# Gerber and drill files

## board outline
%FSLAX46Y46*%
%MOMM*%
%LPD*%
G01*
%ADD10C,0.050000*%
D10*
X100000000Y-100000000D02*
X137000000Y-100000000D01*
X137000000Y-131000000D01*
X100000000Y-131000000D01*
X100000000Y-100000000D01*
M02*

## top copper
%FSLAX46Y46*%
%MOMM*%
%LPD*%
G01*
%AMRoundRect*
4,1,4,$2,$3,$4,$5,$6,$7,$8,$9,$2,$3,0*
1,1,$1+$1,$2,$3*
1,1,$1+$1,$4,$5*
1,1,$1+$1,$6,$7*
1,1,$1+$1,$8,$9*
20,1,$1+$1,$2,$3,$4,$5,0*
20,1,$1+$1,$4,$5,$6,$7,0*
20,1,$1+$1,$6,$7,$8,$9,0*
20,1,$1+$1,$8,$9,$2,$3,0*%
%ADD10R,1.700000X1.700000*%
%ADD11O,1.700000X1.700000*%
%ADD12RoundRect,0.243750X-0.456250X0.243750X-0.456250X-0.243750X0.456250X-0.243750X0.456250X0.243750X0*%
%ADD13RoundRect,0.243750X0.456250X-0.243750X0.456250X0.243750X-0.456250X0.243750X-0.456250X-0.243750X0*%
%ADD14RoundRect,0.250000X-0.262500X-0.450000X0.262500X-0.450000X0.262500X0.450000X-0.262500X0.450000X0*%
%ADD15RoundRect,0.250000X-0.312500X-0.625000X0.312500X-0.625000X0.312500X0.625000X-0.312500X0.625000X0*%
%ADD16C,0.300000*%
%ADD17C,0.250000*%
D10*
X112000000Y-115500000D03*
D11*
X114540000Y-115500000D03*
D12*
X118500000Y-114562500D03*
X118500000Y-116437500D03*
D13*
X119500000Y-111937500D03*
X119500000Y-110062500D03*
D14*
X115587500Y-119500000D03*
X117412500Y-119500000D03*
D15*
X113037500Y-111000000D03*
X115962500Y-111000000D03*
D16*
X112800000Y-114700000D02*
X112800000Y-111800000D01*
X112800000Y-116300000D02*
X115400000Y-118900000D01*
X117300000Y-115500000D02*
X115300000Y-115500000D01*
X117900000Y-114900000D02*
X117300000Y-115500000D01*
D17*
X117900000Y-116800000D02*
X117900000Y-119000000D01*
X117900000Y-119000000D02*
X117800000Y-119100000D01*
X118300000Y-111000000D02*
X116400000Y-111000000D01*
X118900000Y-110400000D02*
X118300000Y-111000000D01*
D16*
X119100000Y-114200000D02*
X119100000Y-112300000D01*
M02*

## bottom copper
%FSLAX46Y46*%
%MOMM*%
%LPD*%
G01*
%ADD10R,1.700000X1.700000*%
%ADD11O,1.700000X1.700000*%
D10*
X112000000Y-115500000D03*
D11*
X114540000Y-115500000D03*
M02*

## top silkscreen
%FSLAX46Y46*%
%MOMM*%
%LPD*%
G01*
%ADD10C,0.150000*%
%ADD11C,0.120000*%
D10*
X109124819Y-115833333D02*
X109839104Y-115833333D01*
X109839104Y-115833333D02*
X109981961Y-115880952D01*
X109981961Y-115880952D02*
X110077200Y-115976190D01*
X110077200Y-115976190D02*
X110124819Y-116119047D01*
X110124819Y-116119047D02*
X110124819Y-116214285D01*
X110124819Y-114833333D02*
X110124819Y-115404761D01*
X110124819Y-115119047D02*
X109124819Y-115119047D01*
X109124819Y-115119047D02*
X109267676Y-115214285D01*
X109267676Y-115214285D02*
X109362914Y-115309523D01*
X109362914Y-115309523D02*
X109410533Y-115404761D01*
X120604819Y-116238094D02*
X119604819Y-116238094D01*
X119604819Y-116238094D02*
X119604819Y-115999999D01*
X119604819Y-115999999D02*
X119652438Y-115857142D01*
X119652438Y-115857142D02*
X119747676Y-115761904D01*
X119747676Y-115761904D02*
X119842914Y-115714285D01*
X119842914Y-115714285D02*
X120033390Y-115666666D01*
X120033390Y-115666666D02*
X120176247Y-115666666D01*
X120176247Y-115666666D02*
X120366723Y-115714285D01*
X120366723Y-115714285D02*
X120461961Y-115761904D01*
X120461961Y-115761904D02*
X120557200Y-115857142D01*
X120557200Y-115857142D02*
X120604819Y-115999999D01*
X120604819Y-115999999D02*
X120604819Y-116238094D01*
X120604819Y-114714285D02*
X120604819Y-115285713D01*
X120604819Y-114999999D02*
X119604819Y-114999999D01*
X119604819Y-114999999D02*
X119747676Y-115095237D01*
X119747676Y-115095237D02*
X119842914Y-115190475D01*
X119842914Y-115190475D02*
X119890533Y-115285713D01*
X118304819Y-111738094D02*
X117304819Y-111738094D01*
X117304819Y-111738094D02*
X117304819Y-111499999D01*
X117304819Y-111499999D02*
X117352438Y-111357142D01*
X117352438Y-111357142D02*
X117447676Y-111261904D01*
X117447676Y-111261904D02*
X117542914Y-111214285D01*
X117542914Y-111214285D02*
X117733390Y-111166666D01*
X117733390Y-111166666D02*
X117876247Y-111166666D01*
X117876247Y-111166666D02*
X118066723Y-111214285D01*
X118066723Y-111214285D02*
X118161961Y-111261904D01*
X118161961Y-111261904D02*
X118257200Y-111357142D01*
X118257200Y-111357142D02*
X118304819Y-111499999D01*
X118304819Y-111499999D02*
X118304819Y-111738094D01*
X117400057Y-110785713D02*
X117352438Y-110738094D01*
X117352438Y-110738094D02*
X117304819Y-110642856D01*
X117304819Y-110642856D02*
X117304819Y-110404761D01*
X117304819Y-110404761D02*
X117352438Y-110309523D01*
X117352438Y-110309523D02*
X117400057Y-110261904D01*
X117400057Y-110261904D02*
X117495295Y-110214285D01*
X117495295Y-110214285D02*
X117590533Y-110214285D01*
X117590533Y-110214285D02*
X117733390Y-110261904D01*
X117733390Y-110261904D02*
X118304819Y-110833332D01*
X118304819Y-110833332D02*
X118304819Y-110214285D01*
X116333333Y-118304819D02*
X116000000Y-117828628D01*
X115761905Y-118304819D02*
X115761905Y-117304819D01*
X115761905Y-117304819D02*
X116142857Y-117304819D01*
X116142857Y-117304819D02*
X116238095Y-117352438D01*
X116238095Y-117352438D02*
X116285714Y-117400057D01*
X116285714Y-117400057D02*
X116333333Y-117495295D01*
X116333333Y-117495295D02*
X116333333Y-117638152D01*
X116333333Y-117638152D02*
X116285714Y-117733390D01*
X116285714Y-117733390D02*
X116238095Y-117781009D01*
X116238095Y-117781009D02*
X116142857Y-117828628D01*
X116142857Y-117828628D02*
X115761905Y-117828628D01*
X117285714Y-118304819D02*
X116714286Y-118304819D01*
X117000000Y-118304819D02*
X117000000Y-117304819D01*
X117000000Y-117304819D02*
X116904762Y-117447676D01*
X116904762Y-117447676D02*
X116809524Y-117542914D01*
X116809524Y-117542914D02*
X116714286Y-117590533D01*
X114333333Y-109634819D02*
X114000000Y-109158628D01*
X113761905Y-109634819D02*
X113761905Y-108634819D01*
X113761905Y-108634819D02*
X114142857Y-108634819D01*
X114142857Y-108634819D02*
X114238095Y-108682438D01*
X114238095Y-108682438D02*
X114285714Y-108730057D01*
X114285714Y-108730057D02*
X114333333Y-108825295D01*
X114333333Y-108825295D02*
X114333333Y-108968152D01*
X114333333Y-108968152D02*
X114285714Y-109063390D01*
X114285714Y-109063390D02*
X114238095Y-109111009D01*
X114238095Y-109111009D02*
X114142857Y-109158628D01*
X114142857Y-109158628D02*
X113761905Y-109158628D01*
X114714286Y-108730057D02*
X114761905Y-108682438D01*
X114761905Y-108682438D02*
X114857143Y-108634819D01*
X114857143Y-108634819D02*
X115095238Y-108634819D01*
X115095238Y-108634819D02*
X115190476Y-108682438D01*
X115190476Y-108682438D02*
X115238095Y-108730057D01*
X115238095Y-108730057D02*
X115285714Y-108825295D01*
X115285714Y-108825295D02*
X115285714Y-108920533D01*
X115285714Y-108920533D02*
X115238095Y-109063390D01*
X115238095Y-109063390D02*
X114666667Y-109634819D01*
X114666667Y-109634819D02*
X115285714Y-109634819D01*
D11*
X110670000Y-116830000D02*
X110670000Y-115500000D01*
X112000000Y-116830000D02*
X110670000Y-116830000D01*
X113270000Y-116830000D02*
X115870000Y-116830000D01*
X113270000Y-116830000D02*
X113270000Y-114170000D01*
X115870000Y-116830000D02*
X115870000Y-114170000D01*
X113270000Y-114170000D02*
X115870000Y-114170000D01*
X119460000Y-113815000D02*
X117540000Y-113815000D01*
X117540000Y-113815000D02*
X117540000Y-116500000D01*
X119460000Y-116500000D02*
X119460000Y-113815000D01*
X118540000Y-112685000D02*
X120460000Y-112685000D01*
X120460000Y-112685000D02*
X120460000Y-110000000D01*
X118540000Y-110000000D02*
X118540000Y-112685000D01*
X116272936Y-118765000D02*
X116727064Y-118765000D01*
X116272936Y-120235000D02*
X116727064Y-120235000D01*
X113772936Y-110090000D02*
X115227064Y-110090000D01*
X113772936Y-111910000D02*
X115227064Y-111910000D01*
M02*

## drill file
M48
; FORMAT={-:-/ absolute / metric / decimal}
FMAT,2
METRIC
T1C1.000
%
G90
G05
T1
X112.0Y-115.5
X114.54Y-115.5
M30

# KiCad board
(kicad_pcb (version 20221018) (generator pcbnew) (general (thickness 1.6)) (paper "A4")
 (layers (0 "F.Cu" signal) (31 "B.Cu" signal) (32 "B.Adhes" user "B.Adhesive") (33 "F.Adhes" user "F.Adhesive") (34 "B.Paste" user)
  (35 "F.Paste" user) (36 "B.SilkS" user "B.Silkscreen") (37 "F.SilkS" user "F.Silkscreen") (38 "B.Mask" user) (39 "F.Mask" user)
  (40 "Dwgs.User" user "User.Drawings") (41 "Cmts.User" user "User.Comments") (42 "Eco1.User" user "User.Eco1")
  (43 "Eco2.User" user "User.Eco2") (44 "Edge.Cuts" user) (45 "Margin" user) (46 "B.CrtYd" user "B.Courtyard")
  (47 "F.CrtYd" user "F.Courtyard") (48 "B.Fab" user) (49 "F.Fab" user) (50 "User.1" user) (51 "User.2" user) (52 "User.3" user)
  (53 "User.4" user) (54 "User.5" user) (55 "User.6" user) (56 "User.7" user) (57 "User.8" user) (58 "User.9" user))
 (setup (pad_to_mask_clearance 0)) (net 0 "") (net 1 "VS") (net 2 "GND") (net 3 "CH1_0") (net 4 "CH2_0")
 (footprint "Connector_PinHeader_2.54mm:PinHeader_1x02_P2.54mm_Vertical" (layer "F.Cu") (at 112 115.5 90)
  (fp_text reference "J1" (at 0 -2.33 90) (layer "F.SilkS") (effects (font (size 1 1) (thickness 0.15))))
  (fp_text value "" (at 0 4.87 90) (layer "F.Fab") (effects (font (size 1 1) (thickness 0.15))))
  (fp_line (start -1.33 -1.33) (end 0 -1.33) (stroke (width 0.12) (type solid)) (layer "F.SilkS"))
  (fp_line (start -1.33 0) (end -1.33 -1.33) (stroke (width 0.12) (type solid)) (layer "F.SilkS"))
  (fp_line (start -1.33 1.27) (end -1.33 3.87) (stroke (width 0.12) (type solid)) (layer "F.SilkS"))
  (fp_line (start -1.33 1.27) (end 1.33 1.27) (stroke (width 0.12) (type solid)) (layer "F.SilkS"))
  (fp_line (start -1.33 3.87) (end 1.33 3.87) (stroke (width 0.12) (type solid)) (layer "F.SilkS"))
  (fp_line (start 1.33 1.27) (end 1.33 3.87) (stroke (width 0.12) (type solid)) (layer "F.SilkS"))
  (pad "1" thru_hole rect (at 0 0 90) (size 1.7 1.7) (drill 1) (layers "*.Cu" "*.Mask") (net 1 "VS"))
  (pad "2" thru_hole oval (at 0 2.54 90) (size 1.7 1.7) (drill 1) (layers "*.Cu" "*.Mask") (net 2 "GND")))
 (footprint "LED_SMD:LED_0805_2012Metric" (layer "F.Cu") (at 118.5 115.5 -90)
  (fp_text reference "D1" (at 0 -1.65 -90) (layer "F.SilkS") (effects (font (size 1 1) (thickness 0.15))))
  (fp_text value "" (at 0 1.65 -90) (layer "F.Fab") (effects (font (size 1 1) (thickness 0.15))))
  (fp_line (start -1.685 -0.96) (end -1.685 0.96) (stroke (width 0.12) (type solid)) (layer "F.SilkS"))
  (fp_line (start -1.685 0.96) (end 1 0.96) (stroke (width 0.12) (type solid)) (layer "F.SilkS"))
  (fp_line (start 1 -0.96) (end -1.685 -0.96) (stroke (width 0.12) (type solid)) (layer "F.SilkS"))
  (pad "1" smd roundrect (at -0.9375 0 270) (size 0.975 1.4) (layers "F.Cu" "F.Paste" "F.Mask") (roundrect_rratio 0.25) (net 2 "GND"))
  (pad "2" smd roundrect (at 0.9375 0 270) (size 0.975 1.4) (layers "F.Cu" "F.Paste" "F.Mask") (roundrect_rratio 0.25) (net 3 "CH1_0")))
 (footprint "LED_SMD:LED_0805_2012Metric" (layer "F.Cu") (at 119.5 111 90)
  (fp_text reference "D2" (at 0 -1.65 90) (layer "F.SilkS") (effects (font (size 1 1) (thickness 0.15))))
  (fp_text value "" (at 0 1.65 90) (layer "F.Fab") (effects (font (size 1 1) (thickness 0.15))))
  (fp_line (start -1.685 -0.96) (end -1.685 0.96) (stroke (width 0.12) (type solid)) (layer "F.SilkS"))
  (fp_line (start -1.685 0.96) (end 1 0.96) (stroke (width 0.12) (type solid)) (layer "F.SilkS"))
  (fp_line (start 1 -0.96) (end -1.685 -0.96) (stroke (width 0.12) (type solid)) (layer "F.SilkS"))
  (pad "1" smd roundrect (at -0.9375 0 90) (size 0.975 1.4) (layers "F.Cu" "F.Paste" "F.Mask") (roundrect_rratio 0.25) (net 2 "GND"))
  (pad "2" smd roundrect (at 0.9375 0 90) (size 0.975 1.4) (layers "F.Cu" "F.Paste" "F.Mask") (roundrect_rratio 0.25) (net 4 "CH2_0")))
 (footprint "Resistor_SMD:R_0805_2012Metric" (layer "F.Cu") (at 116.5 119.5)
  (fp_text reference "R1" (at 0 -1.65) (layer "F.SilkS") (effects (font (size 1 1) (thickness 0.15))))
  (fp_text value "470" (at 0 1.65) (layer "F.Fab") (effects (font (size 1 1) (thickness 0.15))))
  (fp_line (start -0.227064 -0.735) (end 0.227064 -0.735) (stroke (width 0.12) (type solid)) (layer "F.SilkS"))
  (fp_line (start -0.227064 0.735) (end 0.227064 0.735) (stroke (width 0.12) (type solid)) (layer "F.SilkS"))
  (pad "1" smd roundrect (at -0.9125 0) (size 1.025 1.4) (layers "F.Cu" "F.Paste" "F.Mask") (roundrect_rratio 0.243902) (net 1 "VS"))
  (pad "2" smd roundrect (at 0.9125 0) (size 1.025 1.4) (layers "F.Cu" "F.Paste" "F.Mask") (roundrect_rratio 0.243902) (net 3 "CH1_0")))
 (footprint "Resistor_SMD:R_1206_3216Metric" (layer "F.Cu") (at 114.5 111)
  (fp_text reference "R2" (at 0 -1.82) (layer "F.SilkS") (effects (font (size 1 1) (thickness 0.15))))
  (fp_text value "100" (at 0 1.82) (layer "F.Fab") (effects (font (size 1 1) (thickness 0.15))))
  (fp_line (start -0.727064 -0.91) (end 0.727064 -0.91) (stroke (width 0.12) (type solid)) (layer "F.SilkS"))
  (fp_line (start -0.727064 0.91) (end 0.727064 0.91) (stroke (width 0.12) (type solid)) (layer "F.SilkS"))
  (pad "1" smd roundrect (at -1.4625 0) (size 1.125 1.75) (layers "F.Cu" "F.Paste" "F.Mask") (roundrect_rratio 0.222222) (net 1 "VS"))
  (pad "2" smd roundrect (at 1.4625 0) (size 1.125 1.75) (layers "F.Cu" "F.Paste" "F.Mask") (roundrect_rratio 0.222222) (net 4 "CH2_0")))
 (gr_rect (start 100 100) (end 137 131) (stroke (width 0.05) (type default)) (fill none) (layer "Edge.Cuts"))
 (segment (start 112.8 114.7) (end 112.8 111.8) (width 0.3) (layer "F.Cu") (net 1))
 (segment (start 112.8 116.3) (end 115.4 118.9) (width 0.3) (layer "F.Cu") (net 1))
 (segment (start 117.3 115.5) (end 115.3 115.5) (width 0.3) (layer "F.Cu") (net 2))
 (segment (start 117.9 114.9) (end 117.3 115.5) (width 0.3) (layer "F.Cu") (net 2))
 (segment (start 117.9 116.8) (end 117.9 119) (width 0.25) (layer "F.Cu") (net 3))
 (segment (start 117.9 119) (end 117.8 119.1) (width 0.25) (layer "F.Cu") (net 3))
 (segment (start 118.3 111) (end 116.4 111) (width 0.25) (layer "F.Cu") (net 4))
 (segment (start 118.9 110.4) (end 118.3 111) (width 0.25) (layer "F.Cu") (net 4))
 (segment (start 119.1 114.2) (end 119.1 112.3) (width 0.3) (layer "F.Cu") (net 2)))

